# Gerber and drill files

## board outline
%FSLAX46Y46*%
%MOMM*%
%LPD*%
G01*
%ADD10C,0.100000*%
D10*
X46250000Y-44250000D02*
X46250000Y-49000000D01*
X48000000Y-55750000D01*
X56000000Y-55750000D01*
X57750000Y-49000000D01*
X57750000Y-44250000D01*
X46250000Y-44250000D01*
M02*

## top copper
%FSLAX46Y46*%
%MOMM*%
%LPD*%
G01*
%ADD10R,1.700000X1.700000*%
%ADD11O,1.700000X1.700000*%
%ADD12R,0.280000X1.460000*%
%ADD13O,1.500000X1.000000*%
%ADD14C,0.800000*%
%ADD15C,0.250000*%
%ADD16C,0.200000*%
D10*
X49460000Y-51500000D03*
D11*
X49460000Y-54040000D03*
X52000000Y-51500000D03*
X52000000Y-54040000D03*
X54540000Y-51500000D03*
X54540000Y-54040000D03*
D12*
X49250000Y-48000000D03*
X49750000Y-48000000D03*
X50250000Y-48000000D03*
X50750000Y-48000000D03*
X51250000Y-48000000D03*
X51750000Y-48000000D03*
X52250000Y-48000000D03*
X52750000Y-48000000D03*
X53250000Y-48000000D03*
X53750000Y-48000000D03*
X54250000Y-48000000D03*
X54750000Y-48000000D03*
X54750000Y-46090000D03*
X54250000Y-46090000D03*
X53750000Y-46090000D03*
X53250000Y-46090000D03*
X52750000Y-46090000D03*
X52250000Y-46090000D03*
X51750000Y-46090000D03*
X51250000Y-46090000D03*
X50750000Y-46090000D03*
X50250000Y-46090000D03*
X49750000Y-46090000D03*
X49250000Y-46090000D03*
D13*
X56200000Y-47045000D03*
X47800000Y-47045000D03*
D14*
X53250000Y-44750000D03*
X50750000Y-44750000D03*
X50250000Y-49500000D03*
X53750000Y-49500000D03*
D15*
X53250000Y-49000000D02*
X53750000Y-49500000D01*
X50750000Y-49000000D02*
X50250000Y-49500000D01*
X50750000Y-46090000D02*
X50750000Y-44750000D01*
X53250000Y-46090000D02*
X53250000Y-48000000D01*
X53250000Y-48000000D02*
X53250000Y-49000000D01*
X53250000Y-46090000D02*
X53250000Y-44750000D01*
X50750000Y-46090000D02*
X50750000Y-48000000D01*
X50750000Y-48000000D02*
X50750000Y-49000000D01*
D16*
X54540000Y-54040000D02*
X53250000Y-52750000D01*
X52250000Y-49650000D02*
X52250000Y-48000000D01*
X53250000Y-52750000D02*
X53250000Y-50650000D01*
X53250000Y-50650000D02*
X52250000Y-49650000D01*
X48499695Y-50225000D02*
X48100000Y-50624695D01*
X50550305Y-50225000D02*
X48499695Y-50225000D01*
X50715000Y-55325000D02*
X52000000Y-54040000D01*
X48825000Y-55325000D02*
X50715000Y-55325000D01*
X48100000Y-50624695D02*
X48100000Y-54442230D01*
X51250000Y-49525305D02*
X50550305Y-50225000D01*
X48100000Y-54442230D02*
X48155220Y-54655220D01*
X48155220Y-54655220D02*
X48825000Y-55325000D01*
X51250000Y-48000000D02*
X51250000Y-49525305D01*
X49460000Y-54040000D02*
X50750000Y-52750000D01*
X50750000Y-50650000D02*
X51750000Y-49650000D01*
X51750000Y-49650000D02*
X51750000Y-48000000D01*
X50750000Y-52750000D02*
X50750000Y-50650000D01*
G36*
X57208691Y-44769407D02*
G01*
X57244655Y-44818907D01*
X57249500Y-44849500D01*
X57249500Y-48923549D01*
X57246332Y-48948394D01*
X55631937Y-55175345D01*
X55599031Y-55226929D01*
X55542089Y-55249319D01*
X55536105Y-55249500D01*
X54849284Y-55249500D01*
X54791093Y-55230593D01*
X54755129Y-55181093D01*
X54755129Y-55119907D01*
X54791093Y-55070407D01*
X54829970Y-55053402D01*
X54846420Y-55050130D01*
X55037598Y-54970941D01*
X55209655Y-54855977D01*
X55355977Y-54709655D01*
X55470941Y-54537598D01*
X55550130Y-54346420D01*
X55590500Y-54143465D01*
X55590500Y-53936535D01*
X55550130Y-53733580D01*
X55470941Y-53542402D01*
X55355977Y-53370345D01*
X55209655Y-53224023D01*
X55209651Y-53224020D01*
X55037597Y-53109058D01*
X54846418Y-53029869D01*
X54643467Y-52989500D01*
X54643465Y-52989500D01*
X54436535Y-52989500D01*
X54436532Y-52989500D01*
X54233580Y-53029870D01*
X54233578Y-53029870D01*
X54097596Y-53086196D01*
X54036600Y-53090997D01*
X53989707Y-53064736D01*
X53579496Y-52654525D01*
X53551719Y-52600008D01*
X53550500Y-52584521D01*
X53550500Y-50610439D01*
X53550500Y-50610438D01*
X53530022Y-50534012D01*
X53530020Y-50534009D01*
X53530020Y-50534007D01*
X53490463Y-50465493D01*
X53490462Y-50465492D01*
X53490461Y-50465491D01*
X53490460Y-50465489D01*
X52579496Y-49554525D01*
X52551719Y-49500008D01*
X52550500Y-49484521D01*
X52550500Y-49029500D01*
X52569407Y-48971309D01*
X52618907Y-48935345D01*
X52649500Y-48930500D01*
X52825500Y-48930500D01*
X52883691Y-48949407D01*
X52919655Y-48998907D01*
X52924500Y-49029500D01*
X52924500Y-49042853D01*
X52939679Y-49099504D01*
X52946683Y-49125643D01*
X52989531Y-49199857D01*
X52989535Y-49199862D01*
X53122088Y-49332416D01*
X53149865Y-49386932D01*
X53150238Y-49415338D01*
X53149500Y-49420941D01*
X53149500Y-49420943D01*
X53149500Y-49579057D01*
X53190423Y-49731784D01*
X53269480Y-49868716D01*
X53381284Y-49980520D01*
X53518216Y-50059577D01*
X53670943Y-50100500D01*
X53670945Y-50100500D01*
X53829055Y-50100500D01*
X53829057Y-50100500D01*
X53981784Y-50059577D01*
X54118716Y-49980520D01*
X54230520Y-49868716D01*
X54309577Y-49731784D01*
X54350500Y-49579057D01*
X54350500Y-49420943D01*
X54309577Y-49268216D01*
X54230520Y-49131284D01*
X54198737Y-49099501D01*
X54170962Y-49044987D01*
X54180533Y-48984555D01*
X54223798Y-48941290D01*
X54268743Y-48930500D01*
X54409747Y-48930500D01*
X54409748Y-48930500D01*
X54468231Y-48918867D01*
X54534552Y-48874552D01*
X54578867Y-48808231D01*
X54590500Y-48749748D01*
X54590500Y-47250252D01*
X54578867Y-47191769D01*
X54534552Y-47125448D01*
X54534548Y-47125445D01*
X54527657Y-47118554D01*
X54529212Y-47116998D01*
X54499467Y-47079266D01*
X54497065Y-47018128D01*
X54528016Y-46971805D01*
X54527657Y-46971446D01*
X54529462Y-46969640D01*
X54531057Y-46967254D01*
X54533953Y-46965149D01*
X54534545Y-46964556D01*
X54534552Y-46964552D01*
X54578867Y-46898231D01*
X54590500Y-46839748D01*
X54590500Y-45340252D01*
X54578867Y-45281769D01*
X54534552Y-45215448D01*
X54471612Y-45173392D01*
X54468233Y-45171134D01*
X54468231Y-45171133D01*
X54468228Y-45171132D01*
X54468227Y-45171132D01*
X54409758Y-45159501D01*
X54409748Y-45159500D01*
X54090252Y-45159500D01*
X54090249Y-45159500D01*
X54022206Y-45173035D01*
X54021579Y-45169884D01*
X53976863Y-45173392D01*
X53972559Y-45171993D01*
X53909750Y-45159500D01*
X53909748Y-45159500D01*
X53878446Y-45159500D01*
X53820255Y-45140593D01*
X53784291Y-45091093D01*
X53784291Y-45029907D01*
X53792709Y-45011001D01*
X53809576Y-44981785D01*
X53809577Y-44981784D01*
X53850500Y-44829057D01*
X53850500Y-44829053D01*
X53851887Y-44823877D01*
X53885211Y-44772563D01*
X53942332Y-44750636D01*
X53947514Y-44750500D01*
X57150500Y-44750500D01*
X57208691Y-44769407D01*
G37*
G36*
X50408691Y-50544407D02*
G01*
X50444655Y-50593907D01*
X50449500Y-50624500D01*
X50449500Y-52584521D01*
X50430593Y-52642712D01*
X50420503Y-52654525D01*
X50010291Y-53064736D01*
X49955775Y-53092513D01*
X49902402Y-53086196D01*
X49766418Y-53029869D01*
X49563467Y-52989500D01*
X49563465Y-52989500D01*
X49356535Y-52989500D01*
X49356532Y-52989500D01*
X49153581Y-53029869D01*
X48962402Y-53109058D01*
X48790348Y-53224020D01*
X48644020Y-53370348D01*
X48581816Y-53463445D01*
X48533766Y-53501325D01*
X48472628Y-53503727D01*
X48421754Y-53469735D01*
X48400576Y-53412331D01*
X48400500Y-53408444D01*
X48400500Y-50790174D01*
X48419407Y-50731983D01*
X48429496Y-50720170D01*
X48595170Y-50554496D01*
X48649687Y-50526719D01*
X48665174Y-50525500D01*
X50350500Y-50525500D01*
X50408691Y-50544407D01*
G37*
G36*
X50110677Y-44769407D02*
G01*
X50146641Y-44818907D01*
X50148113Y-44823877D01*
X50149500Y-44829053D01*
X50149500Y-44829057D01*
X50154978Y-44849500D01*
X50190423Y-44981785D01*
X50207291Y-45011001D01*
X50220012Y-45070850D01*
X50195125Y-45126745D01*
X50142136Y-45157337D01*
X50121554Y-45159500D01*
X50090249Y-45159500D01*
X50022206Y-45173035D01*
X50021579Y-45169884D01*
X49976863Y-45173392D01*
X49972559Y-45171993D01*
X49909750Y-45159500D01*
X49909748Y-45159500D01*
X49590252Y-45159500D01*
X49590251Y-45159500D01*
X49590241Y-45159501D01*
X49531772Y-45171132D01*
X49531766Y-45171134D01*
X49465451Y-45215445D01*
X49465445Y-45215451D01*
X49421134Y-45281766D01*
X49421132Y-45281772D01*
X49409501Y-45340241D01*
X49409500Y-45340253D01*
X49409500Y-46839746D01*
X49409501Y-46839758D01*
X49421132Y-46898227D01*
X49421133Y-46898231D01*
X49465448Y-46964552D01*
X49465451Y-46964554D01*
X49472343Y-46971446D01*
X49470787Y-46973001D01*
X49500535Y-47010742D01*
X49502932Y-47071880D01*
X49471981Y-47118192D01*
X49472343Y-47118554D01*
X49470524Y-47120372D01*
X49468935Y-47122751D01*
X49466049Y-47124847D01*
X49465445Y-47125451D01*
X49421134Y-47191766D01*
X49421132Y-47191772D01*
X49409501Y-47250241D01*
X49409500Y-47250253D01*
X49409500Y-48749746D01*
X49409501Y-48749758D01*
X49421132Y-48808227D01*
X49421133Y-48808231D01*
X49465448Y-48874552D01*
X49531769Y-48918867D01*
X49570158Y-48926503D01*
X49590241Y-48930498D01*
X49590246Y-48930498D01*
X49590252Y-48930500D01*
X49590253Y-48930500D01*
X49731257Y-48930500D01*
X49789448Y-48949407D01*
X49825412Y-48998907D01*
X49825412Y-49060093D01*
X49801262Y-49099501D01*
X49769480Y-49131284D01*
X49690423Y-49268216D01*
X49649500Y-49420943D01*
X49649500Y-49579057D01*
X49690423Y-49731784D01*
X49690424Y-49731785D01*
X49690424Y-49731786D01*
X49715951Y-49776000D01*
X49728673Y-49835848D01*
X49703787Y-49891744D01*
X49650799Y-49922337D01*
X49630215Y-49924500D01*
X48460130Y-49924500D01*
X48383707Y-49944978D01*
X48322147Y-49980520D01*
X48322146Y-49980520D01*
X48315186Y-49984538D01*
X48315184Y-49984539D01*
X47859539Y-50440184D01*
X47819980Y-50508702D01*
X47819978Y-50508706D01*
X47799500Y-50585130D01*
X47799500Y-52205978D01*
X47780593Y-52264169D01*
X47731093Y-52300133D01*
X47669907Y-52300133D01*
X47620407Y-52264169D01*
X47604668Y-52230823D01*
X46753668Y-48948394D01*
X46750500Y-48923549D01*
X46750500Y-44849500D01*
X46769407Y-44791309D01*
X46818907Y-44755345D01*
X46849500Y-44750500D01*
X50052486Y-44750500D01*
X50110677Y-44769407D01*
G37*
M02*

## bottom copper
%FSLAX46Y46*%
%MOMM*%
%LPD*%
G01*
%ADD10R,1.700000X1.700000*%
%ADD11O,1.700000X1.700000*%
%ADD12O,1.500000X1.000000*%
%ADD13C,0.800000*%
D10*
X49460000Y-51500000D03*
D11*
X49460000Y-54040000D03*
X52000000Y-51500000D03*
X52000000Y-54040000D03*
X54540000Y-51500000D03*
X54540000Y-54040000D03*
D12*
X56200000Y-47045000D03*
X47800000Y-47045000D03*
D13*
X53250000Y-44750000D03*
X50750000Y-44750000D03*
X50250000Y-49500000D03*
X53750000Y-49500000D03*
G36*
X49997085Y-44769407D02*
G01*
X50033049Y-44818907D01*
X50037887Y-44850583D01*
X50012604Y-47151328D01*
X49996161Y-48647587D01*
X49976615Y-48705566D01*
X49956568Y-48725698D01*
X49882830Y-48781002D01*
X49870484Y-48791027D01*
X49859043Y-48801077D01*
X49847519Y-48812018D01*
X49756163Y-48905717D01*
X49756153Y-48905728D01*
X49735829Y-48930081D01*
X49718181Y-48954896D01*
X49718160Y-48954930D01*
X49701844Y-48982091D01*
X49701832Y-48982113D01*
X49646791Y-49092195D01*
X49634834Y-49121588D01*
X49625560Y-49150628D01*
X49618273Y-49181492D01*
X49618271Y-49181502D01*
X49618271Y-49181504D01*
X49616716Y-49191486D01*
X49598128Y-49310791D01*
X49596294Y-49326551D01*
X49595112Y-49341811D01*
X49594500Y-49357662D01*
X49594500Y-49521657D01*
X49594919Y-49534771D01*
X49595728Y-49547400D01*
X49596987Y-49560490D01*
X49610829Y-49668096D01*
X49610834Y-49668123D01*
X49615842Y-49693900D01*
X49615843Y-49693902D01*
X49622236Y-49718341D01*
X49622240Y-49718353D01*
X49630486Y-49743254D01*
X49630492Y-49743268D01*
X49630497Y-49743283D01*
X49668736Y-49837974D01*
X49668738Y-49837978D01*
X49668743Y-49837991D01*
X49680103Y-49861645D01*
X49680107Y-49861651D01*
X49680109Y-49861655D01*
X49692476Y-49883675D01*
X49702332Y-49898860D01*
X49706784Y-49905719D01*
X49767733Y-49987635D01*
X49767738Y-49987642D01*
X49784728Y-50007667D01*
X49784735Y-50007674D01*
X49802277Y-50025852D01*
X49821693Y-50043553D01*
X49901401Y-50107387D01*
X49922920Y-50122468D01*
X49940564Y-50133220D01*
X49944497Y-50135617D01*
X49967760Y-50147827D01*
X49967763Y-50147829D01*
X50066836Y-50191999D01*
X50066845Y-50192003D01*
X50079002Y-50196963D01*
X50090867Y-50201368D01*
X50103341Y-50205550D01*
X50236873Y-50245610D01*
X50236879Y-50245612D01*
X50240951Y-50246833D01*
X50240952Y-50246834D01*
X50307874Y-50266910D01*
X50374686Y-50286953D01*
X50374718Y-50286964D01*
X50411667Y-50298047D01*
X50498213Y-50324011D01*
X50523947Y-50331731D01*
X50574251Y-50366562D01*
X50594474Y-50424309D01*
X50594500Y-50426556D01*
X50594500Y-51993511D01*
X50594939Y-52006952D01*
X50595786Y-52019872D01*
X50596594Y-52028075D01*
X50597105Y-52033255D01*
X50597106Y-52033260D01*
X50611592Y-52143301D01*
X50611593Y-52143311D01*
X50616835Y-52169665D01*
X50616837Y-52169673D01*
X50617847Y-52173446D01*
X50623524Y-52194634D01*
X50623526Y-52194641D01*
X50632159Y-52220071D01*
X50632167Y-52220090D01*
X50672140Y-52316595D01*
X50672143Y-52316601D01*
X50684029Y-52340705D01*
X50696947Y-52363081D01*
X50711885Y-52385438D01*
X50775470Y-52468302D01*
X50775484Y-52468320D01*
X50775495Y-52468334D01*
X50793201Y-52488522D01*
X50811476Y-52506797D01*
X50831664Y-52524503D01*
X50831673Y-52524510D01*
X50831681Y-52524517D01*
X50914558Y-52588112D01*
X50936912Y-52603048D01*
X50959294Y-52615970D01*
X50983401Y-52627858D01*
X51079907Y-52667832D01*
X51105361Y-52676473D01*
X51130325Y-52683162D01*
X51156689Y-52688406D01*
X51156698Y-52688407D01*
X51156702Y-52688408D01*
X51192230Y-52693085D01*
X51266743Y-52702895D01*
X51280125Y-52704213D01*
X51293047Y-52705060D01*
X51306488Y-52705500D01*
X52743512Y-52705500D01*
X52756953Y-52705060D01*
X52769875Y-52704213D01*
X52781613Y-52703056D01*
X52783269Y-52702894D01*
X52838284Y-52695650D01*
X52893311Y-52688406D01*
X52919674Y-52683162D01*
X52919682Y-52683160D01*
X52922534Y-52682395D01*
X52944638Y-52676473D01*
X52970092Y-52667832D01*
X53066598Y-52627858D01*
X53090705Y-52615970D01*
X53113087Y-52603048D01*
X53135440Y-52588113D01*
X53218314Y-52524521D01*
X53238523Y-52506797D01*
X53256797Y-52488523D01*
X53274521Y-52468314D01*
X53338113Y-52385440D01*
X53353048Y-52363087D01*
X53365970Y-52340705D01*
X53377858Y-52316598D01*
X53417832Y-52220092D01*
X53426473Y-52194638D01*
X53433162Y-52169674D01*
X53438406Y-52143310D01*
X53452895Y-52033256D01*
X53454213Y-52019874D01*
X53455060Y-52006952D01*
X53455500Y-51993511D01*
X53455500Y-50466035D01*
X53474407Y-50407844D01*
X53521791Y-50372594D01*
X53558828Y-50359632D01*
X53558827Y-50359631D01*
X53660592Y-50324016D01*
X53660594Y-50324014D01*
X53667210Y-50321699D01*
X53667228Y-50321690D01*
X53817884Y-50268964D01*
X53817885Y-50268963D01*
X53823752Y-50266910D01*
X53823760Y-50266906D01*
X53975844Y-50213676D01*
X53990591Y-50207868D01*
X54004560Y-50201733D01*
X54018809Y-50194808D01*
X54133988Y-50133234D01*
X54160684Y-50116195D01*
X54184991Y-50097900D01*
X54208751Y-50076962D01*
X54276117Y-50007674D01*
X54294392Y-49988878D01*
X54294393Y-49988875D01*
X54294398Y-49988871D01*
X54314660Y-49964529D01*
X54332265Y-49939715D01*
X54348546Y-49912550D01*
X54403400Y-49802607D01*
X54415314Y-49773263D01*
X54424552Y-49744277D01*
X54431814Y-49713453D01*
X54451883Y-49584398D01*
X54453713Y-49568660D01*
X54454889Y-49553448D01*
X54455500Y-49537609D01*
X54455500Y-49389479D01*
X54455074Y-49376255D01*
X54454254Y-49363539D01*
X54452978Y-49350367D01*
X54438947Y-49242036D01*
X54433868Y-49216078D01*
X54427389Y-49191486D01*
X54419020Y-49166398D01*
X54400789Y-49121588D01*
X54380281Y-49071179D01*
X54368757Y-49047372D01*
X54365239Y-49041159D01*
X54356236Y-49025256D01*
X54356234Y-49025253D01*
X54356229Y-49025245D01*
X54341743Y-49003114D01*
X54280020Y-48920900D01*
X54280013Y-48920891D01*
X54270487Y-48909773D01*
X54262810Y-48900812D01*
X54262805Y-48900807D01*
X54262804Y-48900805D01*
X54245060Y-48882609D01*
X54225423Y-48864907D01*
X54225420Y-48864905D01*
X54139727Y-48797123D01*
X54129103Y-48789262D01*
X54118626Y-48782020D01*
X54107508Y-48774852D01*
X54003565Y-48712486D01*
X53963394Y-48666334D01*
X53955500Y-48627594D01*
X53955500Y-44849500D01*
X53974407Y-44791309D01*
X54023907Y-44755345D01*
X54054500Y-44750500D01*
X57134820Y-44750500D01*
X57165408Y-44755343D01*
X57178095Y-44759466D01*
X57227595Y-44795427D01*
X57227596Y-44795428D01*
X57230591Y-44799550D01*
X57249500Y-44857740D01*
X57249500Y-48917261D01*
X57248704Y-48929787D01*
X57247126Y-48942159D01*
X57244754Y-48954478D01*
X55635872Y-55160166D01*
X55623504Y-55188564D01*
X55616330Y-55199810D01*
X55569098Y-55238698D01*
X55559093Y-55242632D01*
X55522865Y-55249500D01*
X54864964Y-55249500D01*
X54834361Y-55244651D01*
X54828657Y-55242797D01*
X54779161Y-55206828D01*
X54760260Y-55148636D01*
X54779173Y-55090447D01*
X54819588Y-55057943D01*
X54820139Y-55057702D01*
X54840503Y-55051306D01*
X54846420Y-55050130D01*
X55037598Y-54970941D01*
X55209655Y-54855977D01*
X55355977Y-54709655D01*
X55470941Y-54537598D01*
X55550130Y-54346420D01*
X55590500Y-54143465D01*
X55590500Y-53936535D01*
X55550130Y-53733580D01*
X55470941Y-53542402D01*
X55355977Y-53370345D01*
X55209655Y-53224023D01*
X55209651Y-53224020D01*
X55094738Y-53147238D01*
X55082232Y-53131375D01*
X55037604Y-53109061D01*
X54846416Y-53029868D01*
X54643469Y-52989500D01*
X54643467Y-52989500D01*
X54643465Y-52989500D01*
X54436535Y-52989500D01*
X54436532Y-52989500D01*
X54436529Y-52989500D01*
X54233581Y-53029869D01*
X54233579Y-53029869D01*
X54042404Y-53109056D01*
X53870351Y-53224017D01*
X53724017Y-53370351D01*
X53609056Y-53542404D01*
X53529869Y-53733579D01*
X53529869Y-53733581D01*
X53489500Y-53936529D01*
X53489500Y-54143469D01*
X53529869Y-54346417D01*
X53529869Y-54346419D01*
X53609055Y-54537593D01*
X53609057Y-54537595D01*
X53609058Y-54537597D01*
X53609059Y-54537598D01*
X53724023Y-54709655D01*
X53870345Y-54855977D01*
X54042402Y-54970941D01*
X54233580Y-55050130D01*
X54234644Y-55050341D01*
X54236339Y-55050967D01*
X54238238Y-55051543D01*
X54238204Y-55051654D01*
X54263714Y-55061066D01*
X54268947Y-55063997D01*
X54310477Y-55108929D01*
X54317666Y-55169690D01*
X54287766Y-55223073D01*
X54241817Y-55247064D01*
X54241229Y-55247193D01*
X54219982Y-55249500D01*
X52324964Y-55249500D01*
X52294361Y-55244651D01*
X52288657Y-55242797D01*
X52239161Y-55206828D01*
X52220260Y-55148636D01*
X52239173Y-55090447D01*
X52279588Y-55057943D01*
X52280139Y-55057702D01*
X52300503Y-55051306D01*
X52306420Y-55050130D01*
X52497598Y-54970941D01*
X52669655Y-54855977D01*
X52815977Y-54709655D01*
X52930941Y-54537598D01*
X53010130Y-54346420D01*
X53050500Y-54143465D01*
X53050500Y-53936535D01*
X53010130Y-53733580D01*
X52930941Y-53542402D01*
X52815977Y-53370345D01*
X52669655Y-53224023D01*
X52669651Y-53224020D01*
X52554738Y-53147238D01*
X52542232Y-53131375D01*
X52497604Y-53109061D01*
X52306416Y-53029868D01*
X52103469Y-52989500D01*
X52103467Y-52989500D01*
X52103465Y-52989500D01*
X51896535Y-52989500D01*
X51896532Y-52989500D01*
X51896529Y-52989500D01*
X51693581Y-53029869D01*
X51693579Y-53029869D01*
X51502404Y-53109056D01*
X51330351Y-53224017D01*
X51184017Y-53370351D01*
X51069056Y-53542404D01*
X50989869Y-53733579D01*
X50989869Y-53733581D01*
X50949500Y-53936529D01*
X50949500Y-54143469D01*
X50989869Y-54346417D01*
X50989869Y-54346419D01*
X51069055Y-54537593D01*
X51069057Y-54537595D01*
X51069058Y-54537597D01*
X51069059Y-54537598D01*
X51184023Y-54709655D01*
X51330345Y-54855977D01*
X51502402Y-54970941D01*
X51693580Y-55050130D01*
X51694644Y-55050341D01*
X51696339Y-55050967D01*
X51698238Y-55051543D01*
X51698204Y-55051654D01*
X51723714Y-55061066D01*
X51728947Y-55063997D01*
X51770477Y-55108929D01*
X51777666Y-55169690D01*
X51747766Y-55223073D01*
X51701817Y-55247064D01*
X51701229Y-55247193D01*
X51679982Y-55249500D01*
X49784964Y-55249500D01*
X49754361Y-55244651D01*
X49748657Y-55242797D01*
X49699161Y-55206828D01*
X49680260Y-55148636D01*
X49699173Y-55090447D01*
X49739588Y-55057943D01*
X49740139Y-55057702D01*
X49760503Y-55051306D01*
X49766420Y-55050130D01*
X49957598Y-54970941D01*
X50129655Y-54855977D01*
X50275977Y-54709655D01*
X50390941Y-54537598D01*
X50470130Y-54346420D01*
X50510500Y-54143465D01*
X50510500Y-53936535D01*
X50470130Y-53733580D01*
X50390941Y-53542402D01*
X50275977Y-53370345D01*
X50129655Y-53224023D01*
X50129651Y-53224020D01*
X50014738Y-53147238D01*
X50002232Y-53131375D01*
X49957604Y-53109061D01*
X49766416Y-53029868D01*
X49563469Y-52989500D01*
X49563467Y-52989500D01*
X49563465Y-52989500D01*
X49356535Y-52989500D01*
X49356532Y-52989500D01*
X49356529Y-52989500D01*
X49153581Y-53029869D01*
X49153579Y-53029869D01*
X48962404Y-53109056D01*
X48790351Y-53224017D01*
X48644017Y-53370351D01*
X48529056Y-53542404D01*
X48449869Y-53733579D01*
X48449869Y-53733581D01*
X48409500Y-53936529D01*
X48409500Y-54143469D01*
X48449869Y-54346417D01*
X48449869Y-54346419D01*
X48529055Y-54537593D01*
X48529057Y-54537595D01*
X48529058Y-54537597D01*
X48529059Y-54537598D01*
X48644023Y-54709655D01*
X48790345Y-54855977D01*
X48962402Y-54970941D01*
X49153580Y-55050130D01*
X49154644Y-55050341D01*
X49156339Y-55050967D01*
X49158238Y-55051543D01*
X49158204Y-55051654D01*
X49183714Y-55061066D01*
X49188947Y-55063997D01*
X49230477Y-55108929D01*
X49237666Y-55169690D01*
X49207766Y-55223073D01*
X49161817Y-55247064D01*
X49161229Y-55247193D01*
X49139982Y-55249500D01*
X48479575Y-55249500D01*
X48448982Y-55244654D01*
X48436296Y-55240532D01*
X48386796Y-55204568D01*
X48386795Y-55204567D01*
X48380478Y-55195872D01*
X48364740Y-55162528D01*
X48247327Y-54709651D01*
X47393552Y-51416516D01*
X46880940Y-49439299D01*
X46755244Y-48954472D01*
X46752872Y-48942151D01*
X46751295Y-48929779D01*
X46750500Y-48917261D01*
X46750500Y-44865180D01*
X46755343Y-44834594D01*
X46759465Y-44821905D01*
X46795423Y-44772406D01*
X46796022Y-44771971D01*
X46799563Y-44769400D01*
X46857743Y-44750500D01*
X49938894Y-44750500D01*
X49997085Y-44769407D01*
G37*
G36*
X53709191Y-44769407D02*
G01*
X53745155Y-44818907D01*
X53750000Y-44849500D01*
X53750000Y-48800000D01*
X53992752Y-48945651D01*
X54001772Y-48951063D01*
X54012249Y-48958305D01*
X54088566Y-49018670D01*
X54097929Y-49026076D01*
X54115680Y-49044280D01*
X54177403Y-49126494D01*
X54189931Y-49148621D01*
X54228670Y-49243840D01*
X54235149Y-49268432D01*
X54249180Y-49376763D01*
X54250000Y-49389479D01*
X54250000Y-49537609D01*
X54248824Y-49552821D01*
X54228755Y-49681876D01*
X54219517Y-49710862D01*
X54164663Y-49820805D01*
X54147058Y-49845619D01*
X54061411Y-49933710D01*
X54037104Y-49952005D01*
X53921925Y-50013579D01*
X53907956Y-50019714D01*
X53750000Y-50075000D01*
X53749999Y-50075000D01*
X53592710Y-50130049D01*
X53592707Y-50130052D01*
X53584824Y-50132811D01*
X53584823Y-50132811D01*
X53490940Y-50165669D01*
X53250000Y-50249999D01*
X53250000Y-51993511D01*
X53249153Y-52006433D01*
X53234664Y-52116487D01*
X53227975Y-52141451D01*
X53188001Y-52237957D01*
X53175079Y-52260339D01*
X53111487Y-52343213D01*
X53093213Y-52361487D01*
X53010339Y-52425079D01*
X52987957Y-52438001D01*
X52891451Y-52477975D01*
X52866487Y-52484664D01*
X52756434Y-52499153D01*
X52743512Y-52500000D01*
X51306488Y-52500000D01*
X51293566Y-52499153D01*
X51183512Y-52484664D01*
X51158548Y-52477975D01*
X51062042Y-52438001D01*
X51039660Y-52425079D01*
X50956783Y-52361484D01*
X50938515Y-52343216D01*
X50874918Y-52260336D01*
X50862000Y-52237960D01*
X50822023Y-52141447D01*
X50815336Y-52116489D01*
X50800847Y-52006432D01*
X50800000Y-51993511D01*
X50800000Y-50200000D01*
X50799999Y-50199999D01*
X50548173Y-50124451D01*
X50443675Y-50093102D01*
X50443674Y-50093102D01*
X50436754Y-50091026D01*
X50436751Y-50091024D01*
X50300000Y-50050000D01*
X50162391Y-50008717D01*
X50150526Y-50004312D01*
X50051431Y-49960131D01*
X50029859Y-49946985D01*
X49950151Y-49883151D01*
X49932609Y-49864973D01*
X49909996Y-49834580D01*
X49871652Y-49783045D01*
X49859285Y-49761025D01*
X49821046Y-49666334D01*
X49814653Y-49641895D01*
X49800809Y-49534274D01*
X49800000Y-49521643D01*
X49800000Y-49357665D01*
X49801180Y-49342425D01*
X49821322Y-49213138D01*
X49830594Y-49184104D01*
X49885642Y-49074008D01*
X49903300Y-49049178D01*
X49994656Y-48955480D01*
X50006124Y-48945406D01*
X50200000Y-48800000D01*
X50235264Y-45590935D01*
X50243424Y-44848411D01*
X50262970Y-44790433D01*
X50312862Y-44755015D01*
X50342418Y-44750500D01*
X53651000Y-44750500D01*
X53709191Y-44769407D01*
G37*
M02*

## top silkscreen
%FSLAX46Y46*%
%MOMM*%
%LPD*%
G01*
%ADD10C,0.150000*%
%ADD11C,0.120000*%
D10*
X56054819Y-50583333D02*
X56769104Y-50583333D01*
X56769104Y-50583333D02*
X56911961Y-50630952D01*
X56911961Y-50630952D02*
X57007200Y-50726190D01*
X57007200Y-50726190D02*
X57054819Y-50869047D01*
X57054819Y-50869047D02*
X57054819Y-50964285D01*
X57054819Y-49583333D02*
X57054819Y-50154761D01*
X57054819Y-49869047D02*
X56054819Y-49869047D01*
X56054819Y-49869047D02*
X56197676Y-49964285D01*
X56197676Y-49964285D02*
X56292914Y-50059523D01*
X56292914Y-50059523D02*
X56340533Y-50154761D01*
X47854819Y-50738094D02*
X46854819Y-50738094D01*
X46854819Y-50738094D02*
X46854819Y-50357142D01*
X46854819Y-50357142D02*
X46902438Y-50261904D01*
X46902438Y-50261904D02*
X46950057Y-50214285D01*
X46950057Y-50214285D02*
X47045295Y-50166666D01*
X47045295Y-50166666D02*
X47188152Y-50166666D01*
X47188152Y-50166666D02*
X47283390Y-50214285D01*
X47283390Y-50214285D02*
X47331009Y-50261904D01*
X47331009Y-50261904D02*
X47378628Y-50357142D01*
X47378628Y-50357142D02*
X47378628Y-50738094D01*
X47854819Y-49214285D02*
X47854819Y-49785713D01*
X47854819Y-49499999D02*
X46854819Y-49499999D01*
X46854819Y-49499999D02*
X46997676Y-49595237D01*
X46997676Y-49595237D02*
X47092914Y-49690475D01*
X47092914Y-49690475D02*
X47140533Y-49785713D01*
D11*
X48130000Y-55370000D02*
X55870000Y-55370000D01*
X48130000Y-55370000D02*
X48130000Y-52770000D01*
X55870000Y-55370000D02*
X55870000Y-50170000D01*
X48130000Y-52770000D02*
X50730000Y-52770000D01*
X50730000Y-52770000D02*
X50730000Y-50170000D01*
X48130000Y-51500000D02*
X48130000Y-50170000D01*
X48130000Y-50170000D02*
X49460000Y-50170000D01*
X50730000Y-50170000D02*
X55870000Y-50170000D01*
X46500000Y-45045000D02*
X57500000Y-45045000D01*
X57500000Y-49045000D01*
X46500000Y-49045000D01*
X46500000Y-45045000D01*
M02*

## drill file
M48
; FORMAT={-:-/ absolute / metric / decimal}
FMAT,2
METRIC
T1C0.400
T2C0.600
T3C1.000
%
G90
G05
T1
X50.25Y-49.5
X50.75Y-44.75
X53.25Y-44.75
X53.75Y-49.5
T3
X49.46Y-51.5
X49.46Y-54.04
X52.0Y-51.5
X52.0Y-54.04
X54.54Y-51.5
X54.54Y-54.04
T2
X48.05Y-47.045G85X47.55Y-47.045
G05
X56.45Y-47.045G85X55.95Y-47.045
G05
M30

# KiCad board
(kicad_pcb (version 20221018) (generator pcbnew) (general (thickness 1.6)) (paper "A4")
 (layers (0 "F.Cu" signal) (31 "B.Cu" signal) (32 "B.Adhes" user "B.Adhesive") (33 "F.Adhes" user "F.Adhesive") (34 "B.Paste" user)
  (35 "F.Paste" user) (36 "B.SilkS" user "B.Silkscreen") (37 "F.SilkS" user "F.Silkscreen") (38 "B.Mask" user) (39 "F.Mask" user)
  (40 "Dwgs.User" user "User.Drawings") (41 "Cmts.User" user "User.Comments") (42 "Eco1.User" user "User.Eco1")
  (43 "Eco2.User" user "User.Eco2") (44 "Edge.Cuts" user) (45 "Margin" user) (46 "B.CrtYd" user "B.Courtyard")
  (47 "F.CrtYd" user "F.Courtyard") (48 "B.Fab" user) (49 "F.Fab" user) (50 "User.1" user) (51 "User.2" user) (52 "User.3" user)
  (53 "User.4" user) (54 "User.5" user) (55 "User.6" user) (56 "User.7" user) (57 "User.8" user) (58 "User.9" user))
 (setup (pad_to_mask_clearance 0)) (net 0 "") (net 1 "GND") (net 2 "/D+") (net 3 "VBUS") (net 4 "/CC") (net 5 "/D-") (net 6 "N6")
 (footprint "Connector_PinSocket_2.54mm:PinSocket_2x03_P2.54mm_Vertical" (layer "F.Cu") (at 49.46 51.5 90)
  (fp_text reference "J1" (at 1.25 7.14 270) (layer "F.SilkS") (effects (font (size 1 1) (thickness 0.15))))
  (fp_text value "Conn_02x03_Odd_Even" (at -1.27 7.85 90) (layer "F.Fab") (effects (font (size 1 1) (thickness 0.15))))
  (fp_line (start -3.87 -1.33) (end -3.87 6.41) (stroke (width 0.12) (type solid)) (layer "F.SilkS"))
  (fp_line (start -3.87 -1.33) (end -1.27 -1.33) (stroke (width 0.12) (type solid)) (layer "F.SilkS"))
  (fp_line (start -3.87 6.41) (end 1.33 6.41) (stroke (width 0.12) (type solid)) (layer "F.SilkS"))
  (fp_line (start -1.27 -1.33) (end -1.27 1.27) (stroke (width 0.12) (type solid)) (layer "F.SilkS"))
  (fp_line (start -1.27 1.27) (end 1.33 1.27) (stroke (width 0.12) (type solid)) (layer "F.SilkS"))
  (fp_line (start 0 -1.33) (end 1.33 -1.33) (stroke (width 0.12) (type solid)) (layer "F.SilkS"))
  (fp_line (start 1.33 -1.33) (end 1.33 0) (stroke (width 0.12) (type solid)) (layer "F.SilkS"))
  (fp_line (start 1.33 1.27) (end 1.33 6.41) (stroke (width 0.12) (type solid)) (layer "F.SilkS"))
  (pad "1" thru_hole rect (at 0 0 90) (size 1.7 1.7) (drill 1) (layers "*.Cu" "*.Mask") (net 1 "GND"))
  (pad "2" thru_hole oval (at -2.54 0 90) (size 1.7 1.7) (drill 1) (layers "*.Cu" "*.Mask") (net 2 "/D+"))
  (pad "3" thru_hole oval (at 0 2.54 90) (size 1.7 1.7) (drill 1) (layers "*.Cu" "*.Mask") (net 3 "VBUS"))
  (pad "4" thru_hole oval (at -2.54 2.54 90) (size 1.7 1.7) (drill 1) (layers "*.Cu" "*.Mask") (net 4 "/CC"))
  (pad "5" thru_hole oval (at 0 5.08 90) (size 1.7 1.7) (drill 1) (layers "*.Cu" "*.Mask") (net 1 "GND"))
  (pad "6" thru_hole oval (at -2.54 5.08 90) (size 1.7 1.7) (drill 1) (layers "*.Cu" "*.Mask") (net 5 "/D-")))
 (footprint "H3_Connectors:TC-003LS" (layer "F.Cu") (at 52 47.045 180)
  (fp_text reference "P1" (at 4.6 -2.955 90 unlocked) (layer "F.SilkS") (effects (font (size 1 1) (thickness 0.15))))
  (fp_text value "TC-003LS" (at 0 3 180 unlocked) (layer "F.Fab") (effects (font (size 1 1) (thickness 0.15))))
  (fp_rect (start -5.5 -2) (end 5.5 2) (stroke (width 0.12) (type default)) (fill none) (layer "F.SilkS"))
  (pad "A1" smd rect (at 2.75 -0.955 180) (size 0.28 1.46) (layers "F.Cu" "F.Paste" "F.Mask") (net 1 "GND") (thermal_bridge_angle 45))
  (pad "A2" smd rect (at 2.25 -0.955 180) (size 0.28 1.46) (layers "F.Cu" "F.Paste" "F.Mask") (thermal_bridge_angle 45))
  (pad "A3" smd rect (at 1.75 -0.955 180) (size 0.28 1.46) (layers "F.Cu" "F.Paste" "F.Mask") (thermal_bridge_angle 45))
  (pad "A4" smd rect (at 1.25 -0.955 180) (size 0.28 1.46) (layers "F.Cu" "F.Paste" "F.Mask") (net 3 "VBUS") (thermal_bridge_angle 45))
  (pad "A5" smd rect (at 0.75 -0.955 180) (size 0.28 1.46) (layers "F.Cu" "F.Paste" "F.Mask") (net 4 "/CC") (thermal_bridge_angle 45))
  (pad "A6" smd rect (at 0.25 -0.955 180) (size 0.28 1.46) (layers "F.Cu" "F.Paste" "F.Mask") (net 2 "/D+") (thermal_bridge_angle 45))
  (pad "A7" smd rect (at -0.25 -0.955 180) (size 0.28 1.46) (layers "F.Cu" "F.Paste" "F.Mask") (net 5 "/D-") (thermal_bridge_angle 45))
  (pad "A8" smd rect (at -0.75 -0.955 180) (size 0.28 1.46) (layers "F.Cu" "F.Paste" "F.Mask") (thermal_bridge_angle 45))
  (pad "A9" smd rect (at -1.25 -0.955 180) (size 0.28 1.46) (layers "F.Cu" "F.Paste" "F.Mask") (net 3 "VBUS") (thermal_bridge_angle 45))
  (pad "A10" smd rect (at -1.75 -0.955 180) (size 0.28 1.46) (layers "F.Cu" "F.Paste" "F.Mask") (thermal_bridge_angle 45))
  (pad "A11" smd rect (at -2.25 -0.955 180) (size 0.28 1.46) (layers "F.Cu" "F.Paste" "F.Mask") (thermal_bridge_angle 45))
  (pad "A12" smd rect (at -2.75 -0.955 180) (size 0.28 1.46) (layers "F.Cu" "F.Paste" "F.Mask") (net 1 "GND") (thermal_bridge_angle 45))
  (pad "B1" smd rect (at -2.75 0.955) (size 0.28 1.46) (layers "F.Cu" "F.Paste" "F.Mask") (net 1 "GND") (thermal_bridge_angle 45))
  (pad "B2" smd rect (at -2.25 0.955) (size 0.28 1.46) (layers "F.Cu" "F.Paste" "F.Mask") (thermal_bridge_angle 45))
  (pad "B3" smd rect (at -1.75 0.955) (size 0.28 1.46) (layers "F.Cu" "F.Paste" "F.Mask") (thermal_bridge_angle 45))
  (pad "B4" smd rect (at -1.25 0.955) (size 0.28 1.46) (layers "F.Cu" "F.Paste" "F.Mask") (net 3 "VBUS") (thermal_bridge_angle 45))
  (pad "B5" smd rect (at -0.75 0.955) (size 0.28 1.46) (layers "F.Cu" "F.Paste" "F.Mask") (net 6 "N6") (thermal_bridge_angle 45))
  (pad "B6" smd rect (at -0.25 0.955) (size 0.28 1.46) (layers "F.Cu" "F.Paste" "F.Mask") (thermal_bridge_angle 45))
  (pad "B7" smd rect (at 0.25 0.955) (size 0.28 1.46) (layers "F.Cu" "F.Paste" "F.Mask") (thermal_bridge_angle 45))
  (pad "B8" smd rect (at 0.75 0.955) (size 0.28 1.46) (layers "F.Cu" "F.Paste" "F.Mask") (thermal_bridge_angle 45))
  (pad "B9" smd rect (at 1.25 0.955) (size 0.28 1.46) (layers "F.Cu" "F.Paste" "F.Mask") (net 3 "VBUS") (thermal_bridge_angle 45))
  (pad "B10" smd rect (at 1.75 0.955) (size 0.28 1.46) (layers "F.Cu" "F.Paste" "F.Mask") (thermal_bridge_angle 45))
  (pad "B11" smd rect (at 2.25 0.955) (size 0.28 1.46) (layers "F.Cu" "F.Paste" "F.Mask") (thermal_bridge_angle 45))
  (pad "B12" smd rect (at 2.75 0.955) (size 0.28 1.46) (layers "F.Cu" "F.Paste" "F.Mask") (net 1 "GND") (thermal_bridge_angle 45))
  (pad "S1" thru_hole oval (at -4.2 0 180) (size 1.5 1) (drill oval 1.1 0.6) (layers "*.Cu" "*.Mask") (remove_unused_layers)
   (keep_end_layers) (zone_layer_connections) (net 1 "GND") (thermal_bridge_angle 45))
  (pad "S1" thru_hole oval (at 4.2 0 180) (size 1.5 1) (drill oval 1.1 0.6) (layers "*.Cu" "*.Mask") (remove_unused_layers)
   (keep_end_layers) (zone_layer_connections) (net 1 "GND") (thermal_bridge_angle 45)))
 (gr_poly
  (pts (xy 46.25 44.25) (xy 46.25 49) (xy 48 55.75) (xy 56 55.75) (xy 57.75 49) (xy 57.75 44.25)) (stroke (width 0.1) (type solid))
  (fill none) (layer "Edge.Cuts"))
 (segment (start 53.25 49) (end 53.75 49.5) (width 0.25) (layer "F.Cu") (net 3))
 (segment (start 50.75 49) (end 50.25 49.5) (width 0.25) (layer "F.Cu") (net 3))
 (segment (start 50.75 46.09) (end 50.75 44.75) (width 0.25) (layer "F.Cu") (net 3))
 (segment (start 53.25 46.09) (end 53.25 48) (width 0.25) (layer "F.Cu") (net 3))
 (segment (start 53.25 48) (end 53.25 49) (width 0.25) (layer "F.Cu") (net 3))
 (segment (start 53.25 46.09) (end 53.25 44.75) (width 0.25) (layer "F.Cu") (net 3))
 (segment (start 50.75 46.09) (end 50.75 48) (width 0.25) (layer "F.Cu") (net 3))
 (segment (start 50.75 48) (end 50.75 49) (width 0.25) (layer "F.Cu") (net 3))
 (via (at 53.25 44.75) (size 0.8) (drill 0.4) (layers "F.Cu" "B.Cu") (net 3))
 (via (at 50.75 44.75) (size 0.8) (drill 0.4) (layers "F.Cu" "B.Cu") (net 3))
 (via (at 50.25 49.5) (size 0.8) (drill 0.4) (layers "F.Cu" "B.Cu") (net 3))
 (via (at 53.75 49.5) (size 0.8) (drill 0.4) (layers "F.Cu" "B.Cu") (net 3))
 (segment (start 54.54 54.04) (end 53.25 52.75) (width 0.2) (layer "F.Cu") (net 5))
 (segment (start 52.25 49.65) (end 52.25 48) (width 0.2) (layer "F.Cu") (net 5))
 (segment (start 53.25 52.75) (end 53.25 50.65) (width 0.2) (layer "F.Cu") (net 5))
 (segment (start 53.25 50.65) (end 52.25 49.65) (width 0.2) (layer "F.Cu") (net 5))
 (segment (start 48.499695 50.225) (end 48.1 50.624695) (width 0.2) (layer "F.Cu") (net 4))
 (segment (start 50.550305 50.225) (end 48.499695 50.225) (width 0.2) (layer "F.Cu") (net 4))
 (segment (start 50.715 55.325) (end 52 54.04) (width 0.2) (layer "F.Cu") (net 4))
 (segment (start 48.825 55.325) (end 50.715 55.325) (width 0.2) (layer "F.Cu") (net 4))
 (segment (start 48.1 50.624695) (end 48.1 54.44223) (width 0.2) (layer "F.Cu") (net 4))
 (segment (start 51.25 49.525305) (end 50.550305 50.225) (width 0.2) (layer "F.Cu") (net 4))
 (segment (start 48.1 54.44223) (end 48.15522 54.65522) (width 0.2) (layer "F.Cu") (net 4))
 (segment (start 48.15522 54.65522) (end 48.825 55.325) (width 0.2) (layer "F.Cu") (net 4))
 (segment (start 51.25 48) (end 51.25 49.525305) (width 0.2) (layer "F.Cu") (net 4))
 (segment (start 49.46 54.04) (end 50.75 52.75) (width 0.2) (layer "F.Cu") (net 2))
 (segment (start 50.75 50.65) (end 51.75 49.65) (width 0.2) (layer "F.Cu") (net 2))
 (segment (start 51.75 49.65) (end 51.75 48) (width 0.2) (layer "F.Cu") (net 2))
 (segment (start 50.75 52.75) (end 50.75 50.65) (width 0.2) (layer "F.Cu") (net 2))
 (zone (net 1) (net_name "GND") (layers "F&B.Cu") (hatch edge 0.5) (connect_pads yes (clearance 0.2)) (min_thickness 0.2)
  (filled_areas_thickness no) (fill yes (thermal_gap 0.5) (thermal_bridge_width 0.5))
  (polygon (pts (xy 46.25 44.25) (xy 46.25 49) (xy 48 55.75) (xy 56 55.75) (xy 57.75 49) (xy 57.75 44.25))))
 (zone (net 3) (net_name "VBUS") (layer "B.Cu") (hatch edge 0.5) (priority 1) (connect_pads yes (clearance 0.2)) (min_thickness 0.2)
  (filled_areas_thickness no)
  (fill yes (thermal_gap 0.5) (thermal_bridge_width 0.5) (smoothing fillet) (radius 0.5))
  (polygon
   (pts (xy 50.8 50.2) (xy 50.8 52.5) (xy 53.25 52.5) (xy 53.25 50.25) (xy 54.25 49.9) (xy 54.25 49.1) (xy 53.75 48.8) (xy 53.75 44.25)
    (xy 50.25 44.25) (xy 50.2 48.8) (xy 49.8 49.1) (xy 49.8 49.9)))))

